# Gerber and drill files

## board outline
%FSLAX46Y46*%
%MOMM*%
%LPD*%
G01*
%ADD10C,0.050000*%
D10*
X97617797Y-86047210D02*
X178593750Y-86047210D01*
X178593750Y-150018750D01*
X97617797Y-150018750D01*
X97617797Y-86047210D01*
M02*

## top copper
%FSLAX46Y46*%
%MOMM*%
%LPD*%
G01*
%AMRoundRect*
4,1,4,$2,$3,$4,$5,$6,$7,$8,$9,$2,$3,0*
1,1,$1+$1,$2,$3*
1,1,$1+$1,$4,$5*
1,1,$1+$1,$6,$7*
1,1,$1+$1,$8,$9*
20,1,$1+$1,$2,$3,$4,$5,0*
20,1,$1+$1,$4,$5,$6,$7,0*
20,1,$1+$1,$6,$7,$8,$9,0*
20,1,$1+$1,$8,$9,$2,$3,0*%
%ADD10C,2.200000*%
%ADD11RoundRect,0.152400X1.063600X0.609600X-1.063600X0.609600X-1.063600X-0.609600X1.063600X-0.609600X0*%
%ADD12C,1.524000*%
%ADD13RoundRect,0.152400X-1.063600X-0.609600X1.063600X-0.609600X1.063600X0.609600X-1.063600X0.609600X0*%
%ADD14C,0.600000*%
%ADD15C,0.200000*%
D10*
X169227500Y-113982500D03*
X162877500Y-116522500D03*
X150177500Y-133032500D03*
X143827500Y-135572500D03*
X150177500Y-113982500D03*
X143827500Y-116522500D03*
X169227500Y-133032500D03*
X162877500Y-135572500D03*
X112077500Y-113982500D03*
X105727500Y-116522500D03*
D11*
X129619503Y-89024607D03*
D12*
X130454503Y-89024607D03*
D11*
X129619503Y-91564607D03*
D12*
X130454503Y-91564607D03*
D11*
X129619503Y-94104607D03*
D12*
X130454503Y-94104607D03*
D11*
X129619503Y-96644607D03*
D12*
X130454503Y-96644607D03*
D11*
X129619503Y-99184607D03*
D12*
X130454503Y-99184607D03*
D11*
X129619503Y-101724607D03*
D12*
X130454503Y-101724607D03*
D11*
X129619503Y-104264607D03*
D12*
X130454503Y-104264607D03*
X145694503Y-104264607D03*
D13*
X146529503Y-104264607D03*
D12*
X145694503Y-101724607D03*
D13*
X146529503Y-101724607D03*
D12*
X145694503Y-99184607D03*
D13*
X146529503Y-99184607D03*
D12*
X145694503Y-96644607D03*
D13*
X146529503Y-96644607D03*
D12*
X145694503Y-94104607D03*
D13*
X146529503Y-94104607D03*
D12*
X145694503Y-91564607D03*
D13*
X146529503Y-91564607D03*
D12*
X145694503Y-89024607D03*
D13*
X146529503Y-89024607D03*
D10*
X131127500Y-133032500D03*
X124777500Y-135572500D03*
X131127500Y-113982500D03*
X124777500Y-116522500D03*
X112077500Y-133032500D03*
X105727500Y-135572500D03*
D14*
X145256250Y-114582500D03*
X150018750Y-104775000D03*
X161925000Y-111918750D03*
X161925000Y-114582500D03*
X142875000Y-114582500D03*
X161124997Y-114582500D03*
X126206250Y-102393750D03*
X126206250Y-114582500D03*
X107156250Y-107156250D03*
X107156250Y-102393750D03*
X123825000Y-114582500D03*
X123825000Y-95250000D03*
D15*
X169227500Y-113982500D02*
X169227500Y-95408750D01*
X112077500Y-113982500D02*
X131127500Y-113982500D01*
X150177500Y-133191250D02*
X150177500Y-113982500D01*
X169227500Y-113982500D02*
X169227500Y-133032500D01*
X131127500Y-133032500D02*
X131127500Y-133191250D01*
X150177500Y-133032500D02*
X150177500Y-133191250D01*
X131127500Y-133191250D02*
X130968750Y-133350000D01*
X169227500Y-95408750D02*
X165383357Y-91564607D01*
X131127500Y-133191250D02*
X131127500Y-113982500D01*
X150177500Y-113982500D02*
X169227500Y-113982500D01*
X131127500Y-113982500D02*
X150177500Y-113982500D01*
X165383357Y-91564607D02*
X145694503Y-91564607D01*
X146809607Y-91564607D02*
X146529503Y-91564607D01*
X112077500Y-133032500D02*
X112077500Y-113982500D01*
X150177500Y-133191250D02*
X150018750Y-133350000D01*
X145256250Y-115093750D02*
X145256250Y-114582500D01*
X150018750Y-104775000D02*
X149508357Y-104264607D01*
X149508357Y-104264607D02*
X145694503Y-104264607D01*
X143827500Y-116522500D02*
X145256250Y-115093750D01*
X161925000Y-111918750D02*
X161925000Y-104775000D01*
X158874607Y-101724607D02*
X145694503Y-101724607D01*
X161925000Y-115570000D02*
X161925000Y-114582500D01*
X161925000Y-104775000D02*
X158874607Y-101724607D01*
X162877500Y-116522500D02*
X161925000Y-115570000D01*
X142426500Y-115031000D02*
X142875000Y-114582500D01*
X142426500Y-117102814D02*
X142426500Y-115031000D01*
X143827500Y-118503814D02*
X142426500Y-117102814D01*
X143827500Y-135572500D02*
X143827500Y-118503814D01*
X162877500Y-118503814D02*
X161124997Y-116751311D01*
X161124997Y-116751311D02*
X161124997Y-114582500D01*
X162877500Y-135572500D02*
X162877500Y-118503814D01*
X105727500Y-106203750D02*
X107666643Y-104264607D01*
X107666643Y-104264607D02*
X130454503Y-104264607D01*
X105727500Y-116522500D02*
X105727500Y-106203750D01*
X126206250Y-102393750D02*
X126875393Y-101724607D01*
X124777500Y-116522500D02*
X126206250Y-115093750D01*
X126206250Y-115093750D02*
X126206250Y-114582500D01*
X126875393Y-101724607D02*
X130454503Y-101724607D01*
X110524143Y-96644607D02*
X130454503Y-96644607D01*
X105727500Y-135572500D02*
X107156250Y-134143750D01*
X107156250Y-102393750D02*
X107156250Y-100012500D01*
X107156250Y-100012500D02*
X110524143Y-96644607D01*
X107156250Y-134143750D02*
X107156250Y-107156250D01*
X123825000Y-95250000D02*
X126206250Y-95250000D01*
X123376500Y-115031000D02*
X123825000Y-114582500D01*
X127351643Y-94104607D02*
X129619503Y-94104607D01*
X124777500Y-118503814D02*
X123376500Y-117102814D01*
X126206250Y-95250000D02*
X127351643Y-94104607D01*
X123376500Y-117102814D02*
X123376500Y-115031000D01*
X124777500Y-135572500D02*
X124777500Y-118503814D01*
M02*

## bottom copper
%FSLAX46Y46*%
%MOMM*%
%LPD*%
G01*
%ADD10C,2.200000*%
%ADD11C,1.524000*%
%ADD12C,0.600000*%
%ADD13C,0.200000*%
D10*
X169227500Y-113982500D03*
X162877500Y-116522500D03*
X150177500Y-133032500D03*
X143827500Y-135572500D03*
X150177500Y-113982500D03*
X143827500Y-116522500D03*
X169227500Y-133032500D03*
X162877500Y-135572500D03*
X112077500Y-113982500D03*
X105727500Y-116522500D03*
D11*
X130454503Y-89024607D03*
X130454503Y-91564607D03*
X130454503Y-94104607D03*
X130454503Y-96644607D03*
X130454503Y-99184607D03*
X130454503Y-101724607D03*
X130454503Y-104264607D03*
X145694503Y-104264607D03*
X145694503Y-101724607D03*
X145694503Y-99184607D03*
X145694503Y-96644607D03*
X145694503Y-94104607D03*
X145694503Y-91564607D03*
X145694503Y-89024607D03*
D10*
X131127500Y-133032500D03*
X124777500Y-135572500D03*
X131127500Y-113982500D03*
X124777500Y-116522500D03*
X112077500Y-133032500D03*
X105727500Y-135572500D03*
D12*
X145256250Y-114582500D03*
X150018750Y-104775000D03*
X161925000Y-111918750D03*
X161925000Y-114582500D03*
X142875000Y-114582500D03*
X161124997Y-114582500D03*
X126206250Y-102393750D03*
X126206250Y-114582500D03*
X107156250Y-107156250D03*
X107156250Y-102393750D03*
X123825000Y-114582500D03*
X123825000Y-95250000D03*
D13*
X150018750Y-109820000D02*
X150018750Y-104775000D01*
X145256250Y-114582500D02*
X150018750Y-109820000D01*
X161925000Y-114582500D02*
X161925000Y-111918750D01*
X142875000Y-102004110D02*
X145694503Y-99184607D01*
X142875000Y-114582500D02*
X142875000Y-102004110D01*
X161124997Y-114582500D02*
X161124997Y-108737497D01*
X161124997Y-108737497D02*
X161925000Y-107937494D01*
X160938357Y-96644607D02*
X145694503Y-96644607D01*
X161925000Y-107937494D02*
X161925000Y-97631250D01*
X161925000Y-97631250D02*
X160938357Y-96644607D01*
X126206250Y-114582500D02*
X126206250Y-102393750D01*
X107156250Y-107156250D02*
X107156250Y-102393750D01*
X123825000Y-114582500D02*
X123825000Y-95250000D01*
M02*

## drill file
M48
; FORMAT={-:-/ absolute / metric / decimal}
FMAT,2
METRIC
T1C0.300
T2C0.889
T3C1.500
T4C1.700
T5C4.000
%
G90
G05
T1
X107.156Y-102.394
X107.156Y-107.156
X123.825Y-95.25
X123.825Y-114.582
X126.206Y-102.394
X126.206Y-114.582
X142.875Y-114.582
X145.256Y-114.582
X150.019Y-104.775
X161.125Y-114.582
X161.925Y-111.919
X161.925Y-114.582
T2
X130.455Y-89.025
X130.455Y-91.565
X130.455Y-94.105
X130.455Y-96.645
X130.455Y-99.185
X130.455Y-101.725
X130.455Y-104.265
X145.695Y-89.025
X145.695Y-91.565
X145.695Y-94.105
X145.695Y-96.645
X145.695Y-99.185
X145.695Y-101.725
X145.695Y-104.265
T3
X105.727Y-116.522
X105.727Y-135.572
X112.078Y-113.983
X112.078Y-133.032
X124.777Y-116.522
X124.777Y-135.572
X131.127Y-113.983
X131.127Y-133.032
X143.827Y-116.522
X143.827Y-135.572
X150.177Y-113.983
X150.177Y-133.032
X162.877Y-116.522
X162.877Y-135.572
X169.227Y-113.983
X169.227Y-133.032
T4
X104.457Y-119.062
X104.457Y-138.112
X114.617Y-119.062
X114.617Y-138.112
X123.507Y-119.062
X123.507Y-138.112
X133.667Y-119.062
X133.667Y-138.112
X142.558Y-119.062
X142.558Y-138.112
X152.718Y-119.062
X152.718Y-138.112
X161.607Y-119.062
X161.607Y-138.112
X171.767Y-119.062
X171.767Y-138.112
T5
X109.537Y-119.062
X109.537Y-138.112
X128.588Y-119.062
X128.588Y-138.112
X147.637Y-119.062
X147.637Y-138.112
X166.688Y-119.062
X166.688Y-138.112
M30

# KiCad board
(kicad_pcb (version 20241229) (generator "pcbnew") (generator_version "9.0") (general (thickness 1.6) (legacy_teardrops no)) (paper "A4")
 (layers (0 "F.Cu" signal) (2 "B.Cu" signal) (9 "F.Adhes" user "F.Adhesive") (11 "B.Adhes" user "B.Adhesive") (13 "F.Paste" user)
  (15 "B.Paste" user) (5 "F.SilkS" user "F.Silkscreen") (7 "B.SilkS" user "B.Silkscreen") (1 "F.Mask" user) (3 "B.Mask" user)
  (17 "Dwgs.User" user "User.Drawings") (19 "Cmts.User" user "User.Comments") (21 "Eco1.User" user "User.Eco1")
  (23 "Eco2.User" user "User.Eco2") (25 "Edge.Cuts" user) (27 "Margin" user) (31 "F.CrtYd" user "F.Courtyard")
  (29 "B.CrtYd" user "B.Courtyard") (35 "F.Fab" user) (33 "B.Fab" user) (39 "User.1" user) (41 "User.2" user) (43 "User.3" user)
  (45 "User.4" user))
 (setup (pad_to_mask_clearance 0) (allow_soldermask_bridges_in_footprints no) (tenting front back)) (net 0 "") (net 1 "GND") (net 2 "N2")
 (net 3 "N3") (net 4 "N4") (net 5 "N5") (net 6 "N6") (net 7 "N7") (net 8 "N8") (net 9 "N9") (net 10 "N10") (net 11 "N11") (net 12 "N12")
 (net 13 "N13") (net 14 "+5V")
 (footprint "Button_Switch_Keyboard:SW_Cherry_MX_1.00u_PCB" (layer "F.Cu") (at 169.2275 113.9825)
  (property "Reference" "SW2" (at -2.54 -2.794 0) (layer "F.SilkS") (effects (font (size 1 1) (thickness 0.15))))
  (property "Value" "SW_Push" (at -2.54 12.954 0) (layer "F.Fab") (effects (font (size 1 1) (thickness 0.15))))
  (pad "" np_thru_hole circle (at -7.62 5.08) (size 1.7 1.7) (drill 1.7) (layers "*.Cu" "*.Mask"))
  (pad "" np_thru_hole circle (at -2.54 5.08) (size 4 4) (drill 4) (layers "*.Cu" "*.Mask"))
  (pad "" np_thru_hole circle (at 2.54 5.08) (size 1.7 1.7) (drill 1.7) (layers "*.Cu" "*.Mask"))
  (pad "1" thru_hole circle (at 0 0) (size 2.2 2.2) (drill 1.5) (layers "*.Cu" "*.Mask") (remove_unused_layers no) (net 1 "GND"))
  (pad "2" thru_hole circle (at -6.35 2.54) (size 2.2 2.2) (drill 1.5) (layers "*.Cu" "*.Mask") (remove_unused_layers no) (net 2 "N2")))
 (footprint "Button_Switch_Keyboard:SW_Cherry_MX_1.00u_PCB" (layer "F.Cu") (at 150.1775 133.0325)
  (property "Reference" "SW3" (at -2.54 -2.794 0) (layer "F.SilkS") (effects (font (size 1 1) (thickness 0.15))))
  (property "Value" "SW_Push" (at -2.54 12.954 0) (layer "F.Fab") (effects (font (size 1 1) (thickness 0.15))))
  (pad "" np_thru_hole circle (at -7.62 5.08) (size 1.7 1.7) (drill 1.7) (layers "*.Cu" "*.Mask"))
  (pad "" np_thru_hole circle (at -2.54 5.08) (size 4 4) (drill 4) (layers "*.Cu" "*.Mask"))
  (pad "" np_thru_hole circle (at 2.54 5.08) (size 1.7 1.7) (drill 1.7) (layers "*.Cu" "*.Mask"))
  (pad "1" thru_hole circle (at 0 0) (size 2.2 2.2) (drill 1.5) (layers "*.Cu" "*.Mask") (remove_unused_layers no) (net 1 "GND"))
  (pad "2" thru_hole circle (at -6.35 2.54) (size 2.2 2.2) (drill 1.5) (layers "*.Cu" "*.Mask") (remove_unused_layers no) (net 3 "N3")))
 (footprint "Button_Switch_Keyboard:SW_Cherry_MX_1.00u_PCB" (layer "F.Cu") (at 150.1775 113.9825)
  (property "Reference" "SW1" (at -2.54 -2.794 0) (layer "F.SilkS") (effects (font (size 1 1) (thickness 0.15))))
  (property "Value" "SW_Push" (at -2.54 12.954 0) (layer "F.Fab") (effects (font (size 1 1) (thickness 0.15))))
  (pad "" np_thru_hole circle (at -7.62 5.08) (size 1.7 1.7) (drill 1.7) (layers "*.Cu" "*.Mask"))
  (pad "" np_thru_hole circle (at -2.54 5.08) (size 4 4) (drill 4) (layers "*.Cu" "*.Mask"))
  (pad "" np_thru_hole circle (at 2.54 5.08) (size 1.7 1.7) (drill 1.7) (layers "*.Cu" "*.Mask"))
  (pad "1" thru_hole circle (at 0 0) (size 2.2 2.2) (drill 1.5) (layers "*.Cu" "*.Mask") (remove_unused_layers no) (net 1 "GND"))
  (pad "2" thru_hole circle (at -6.35 2.54) (size 2.2 2.2) (drill 1.5) (layers "*.Cu" "*.Mask") (remove_unused_layers no) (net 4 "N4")))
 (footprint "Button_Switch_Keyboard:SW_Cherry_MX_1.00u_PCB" (layer "F.Cu") (at 169.2275 133.0325)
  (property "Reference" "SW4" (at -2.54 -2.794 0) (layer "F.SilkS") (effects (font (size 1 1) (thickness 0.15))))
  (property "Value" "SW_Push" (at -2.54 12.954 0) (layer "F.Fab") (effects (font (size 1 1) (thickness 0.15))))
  (pad "" np_thru_hole circle (at -7.62 5.08) (size 1.7 1.7) (drill 1.7) (layers "*.Cu" "*.Mask"))
  (pad "" np_thru_hole circle (at -2.54 5.08) (size 4 4) (drill 4) (layers "*.Cu" "*.Mask"))
  (pad "" np_thru_hole circle (at 2.54 5.08) (size 1.7 1.7) (drill 1.7) (layers "*.Cu" "*.Mask"))
  (pad "1" thru_hole circle (at 0 0) (size 2.2 2.2) (drill 1.5) (layers "*.Cu" "*.Mask") (remove_unused_layers no) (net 1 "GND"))
  (pad "2" thru_hole circle (at -6.35 2.54) (size 2.2 2.2) (drill 1.5) (layers "*.Cu" "*.Mask") (remove_unused_layers no) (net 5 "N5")))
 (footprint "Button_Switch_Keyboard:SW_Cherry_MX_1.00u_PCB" (layer "F.Cu") (at 112.0775 113.9825)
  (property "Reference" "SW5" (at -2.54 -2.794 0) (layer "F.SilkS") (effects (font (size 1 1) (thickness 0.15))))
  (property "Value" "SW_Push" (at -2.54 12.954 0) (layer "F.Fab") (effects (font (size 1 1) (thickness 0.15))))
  (pad "" np_thru_hole circle (at -7.62 5.08) (size 1.7 1.7) (drill 1.7) (layers "*.Cu" "*.Mask"))
  (pad "" np_thru_hole circle (at -2.54 5.08) (size 4 4) (drill 4) (layers "*.Cu" "*.Mask"))
  (pad "" np_thru_hole circle (at 2.54 5.08) (size 1.7 1.7) (drill 1.7) (layers "*.Cu" "*.Mask"))
  (pad "1" thru_hole circle (at 0 0) (size 2.2 2.2) (drill 1.5) (layers "*.Cu" "*.Mask") (remove_unused_layers no) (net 1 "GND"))
  (pad "2" thru_hole circle (at -6.35 2.54) (size 2.2 2.2) (drill 1.5) (layers "*.Cu" "*.Mask") (remove_unused_layers no) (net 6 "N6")))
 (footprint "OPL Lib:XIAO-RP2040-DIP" (layer "F.Cu") (at 138.074503 96.644607)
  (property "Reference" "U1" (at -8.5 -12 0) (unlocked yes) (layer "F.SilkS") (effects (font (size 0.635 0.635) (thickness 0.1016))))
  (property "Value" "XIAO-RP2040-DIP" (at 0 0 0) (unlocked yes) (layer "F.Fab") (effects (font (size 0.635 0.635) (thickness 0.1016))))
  (pad "1" smd roundrect (at -8.455 -7.62 180) (size 2.432 1.524) (layers "F.Cu" "F.Mask") (roundrect_rratio 0.1) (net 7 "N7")
   (thermal_bridge_angle 45))
  (pad "1" thru_hole circle (at -7.62 -7.62 180) (size 1.524 1.524) (drill 0.889) (layers "*.Cu" "*.Mask") (remove_unused_layers no)
   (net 7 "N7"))
  (pad "2" smd roundrect (at -8.455 -5.08 180) (size 2.432 1.524) (layers "F.Cu" "F.Mask") (roundrect_rratio 0.1) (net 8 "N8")
   (thermal_bridge_angle 45))
  (pad "2" thru_hole circle (at -7.62 -5.08 180) (size 1.524 1.524) (drill 0.889) (layers "*.Cu" "*.Mask") (remove_unused_layers no)
   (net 8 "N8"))
  (pad "3" smd roundrect (at -8.455 -2.54 180) (size 2.432 1.524) (layers "F.Cu" "F.Mask") (roundrect_rratio 0.1) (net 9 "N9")
   (thermal_bridge_angle 45))
  (pad "3" thru_hole circle (at -7.62 -2.54 180) (size 1.524 1.524) (drill 0.889) (layers "*.Cu" "*.Mask") (remove_unused_layers no)
   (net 9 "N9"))
  (pad "4" smd roundrect (at -8.455 0 180) (size 2.432 1.524) (layers "F.Cu" "F.Mask") (roundrect_rratio 0.1) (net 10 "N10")
   (thermal_bridge_angle 45))
  (pad "4" thru_hole circle (at -7.62 0 180) (size 1.524 1.524) (drill 0.889) (layers "*.Cu" "*.Mask") (remove_unused_layers no)
   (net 10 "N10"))
  (pad "5" smd roundrect (at -8.455 2.54 180) (size 2.432 1.524) (layers "F.Cu" "F.Mask") (roundrect_rratio 0.1) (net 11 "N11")
   (thermal_bridge_angle 45))
  (pad "5" thru_hole circle (at -7.62 2.54 180) (size 1.524 1.524) (drill 0.889) (layers "*.Cu" "*.Mask") (remove_unused_layers no)
   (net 11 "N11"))
  (pad "6" smd roundrect (at -8.455 5.08 180) (size 2.432 1.524) (layers "F.Cu" "F.Mask") (roundrect_rratio 0.1) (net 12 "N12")
   (thermal_bridge_angle 45))
  (pad "6" thru_hole circle (at -7.62 5.08 180) (size 1.524 1.524) (drill 0.889) (layers "*.Cu" "*.Mask") (remove_unused_layers no)
   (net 12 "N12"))
  (pad "7" smd roundrect (at -8.455 7.62 180) (size 2.432 1.524) (layers "F.Cu" "F.Mask") (roundrect_rratio 0.1) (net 6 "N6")
   (thermal_bridge_angle 45))
  (pad "7" thru_hole circle (at -7.62 7.62 180) (size 1.524 1.524) (drill 0.889) (layers "*.Cu" "*.Mask") (remove_unused_layers no)
   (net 6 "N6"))
  (pad "8" thru_hole circle (at 7.62 7.62) (size 1.524 1.524) (drill 0.889) (layers "*.Cu" "*.Mask") (remove_unused_layers no) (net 4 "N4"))
  (pad "8" smd roundrect (at 8.455 7.62) (size 2.432 1.524) (layers "F.Cu" "F.Mask") (roundrect_rratio 0.1) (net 4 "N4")
   (thermal_bridge_angle 45))
  (pad "9" thru_hole circle (at 7.62 5.08) (size 1.524 1.524) (drill 0.889) (layers "*.Cu" "*.Mask") (remove_unused_layers no) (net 2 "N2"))
  (pad "9" smd roundrect (at 8.455 5.08) (size 2.432 1.524) (layers "F.Cu" "F.Mask") (roundrect_rratio 0.1) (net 2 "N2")
   (thermal_bridge_angle 45))
  (pad "10" thru_hole circle (at 7.62 2.54) (size 1.524 1.524) (drill 0.889) (layers "*.Cu" "*.Mask") (remove_unused_layers no) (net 3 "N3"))
  (pad "10" smd roundrect (at 8.455 2.54) (size 2.432 1.524) (layers "F.Cu" "F.Mask") (roundrect_rratio 0.1) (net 3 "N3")
   (thermal_bridge_angle 45))
  (pad "11" thru_hole circle (at 7.62 0) (size 1.524 1.524) (drill 0.889) (layers "*.Cu" "*.Mask") (remove_unused_layers no) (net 5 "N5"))
  (pad "11" smd roundrect (at 8.455 0) (size 2.432 1.524) (layers "F.Cu" "F.Mask") (roundrect_rratio 0.1) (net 5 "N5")
   (thermal_bridge_angle 45))
  (pad "12" thru_hole circle (at 7.62 -2.54) (size 1.524 1.524) (drill 0.889) (layers "*.Cu" "*.Mask") (remove_unused_layers no)
   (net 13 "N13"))
  (pad "12" smd roundrect (at 8.455 -2.54) (size 2.432 1.524) (layers "F.Cu" "F.Mask") (roundrect_rratio 0.1) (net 13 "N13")
   (thermal_bridge_angle 45))
  (pad "13" thru_hole circle (at 7.62 -5.08) (size 1.524 1.524) (drill 0.889) (layers "*.Cu" "*.Mask") (remove_unused_layers no)
   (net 1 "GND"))
  (pad "13" smd roundrect (at 8.455 -5.08) (size 2.432 1.524) (layers "F.Cu" "F.Mask") (roundrect_rratio 0.1) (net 1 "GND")
   (thermal_bridge_angle 45))
  (pad "14" thru_hole circle (at 7.62 -7.62) (size 1.524 1.524) (drill 0.889) (layers "*.Cu" "*.Mask") (remove_unused_layers no)
   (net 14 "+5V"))
  (pad "14" smd roundrect (at 8.455 -7.62) (size 2.432 1.524) (layers "F.Cu" "F.Mask") (roundrect_rratio 0.1) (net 14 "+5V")
   (thermal_bridge_angle 45)))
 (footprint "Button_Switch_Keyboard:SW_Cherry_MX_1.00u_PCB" (layer "F.Cu") (at 131.1275 133.0325)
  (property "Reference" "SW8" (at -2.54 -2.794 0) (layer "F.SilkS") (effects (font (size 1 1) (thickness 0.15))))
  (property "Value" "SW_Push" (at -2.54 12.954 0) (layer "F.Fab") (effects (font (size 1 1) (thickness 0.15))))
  (pad "" np_thru_hole circle (at -7.62 5.08) (size 1.7 1.7) (drill 1.7) (layers "*.Cu" "*.Mask"))
  (pad "" np_thru_hole circle (at -2.54 5.08) (size 4 4) (drill 4) (layers "*.Cu" "*.Mask"))
  (pad "" np_thru_hole circle (at 2.54 5.08) (size 1.7 1.7) (drill 1.7) (layers "*.Cu" "*.Mask"))
  (pad "1" thru_hole circle (at 0 0) (size 2.2 2.2) (drill 1.5) (layers "*.Cu" "*.Mask") (remove_unused_layers no) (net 1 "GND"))
  (pad "2" thru_hole circle (at -6.35 2.54) (size 2.2 2.2) (drill 1.5) (layers "*.Cu" "*.Mask") (remove_unused_layers no) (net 9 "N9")))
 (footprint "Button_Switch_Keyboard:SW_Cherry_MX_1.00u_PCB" (layer "F.Cu") (at 131.1275 113.9825)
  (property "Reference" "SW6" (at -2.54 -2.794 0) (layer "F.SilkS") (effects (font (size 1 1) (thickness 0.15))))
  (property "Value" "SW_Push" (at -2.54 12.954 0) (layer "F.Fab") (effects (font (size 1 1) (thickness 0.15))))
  (pad "" np_thru_hole circle (at -7.62 5.08) (size 1.7 1.7) (drill 1.7) (layers "*.Cu" "*.Mask"))
  (pad "" np_thru_hole circle (at -2.54 5.08) (size 4 4) (drill 4) (layers "*.Cu" "*.Mask"))
  (pad "" np_thru_hole circle (at 2.54 5.08) (size 1.7 1.7) (drill 1.7) (layers "*.Cu" "*.Mask"))
  (pad "1" thru_hole circle (at 0 0) (size 2.2 2.2) (drill 1.5) (layers "*.Cu" "*.Mask") (remove_unused_layers no) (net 1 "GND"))
  (pad "2" thru_hole circle (at -6.35 2.54) (size 2.2 2.2) (drill 1.5) (layers "*.Cu" "*.Mask") (remove_unused_layers no) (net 12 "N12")))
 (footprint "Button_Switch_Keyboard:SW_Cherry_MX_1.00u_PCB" (layer "F.Cu") (at 112.0775 133.0325)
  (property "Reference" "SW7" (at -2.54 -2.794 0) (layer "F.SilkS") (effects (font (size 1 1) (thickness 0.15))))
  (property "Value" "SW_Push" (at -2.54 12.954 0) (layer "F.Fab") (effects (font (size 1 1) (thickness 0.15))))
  (pad "" np_thru_hole circle (at -7.62 5.08) (size 1.7 1.7) (drill 1.7) (layers "*.Cu" "*.Mask"))
  (pad "" np_thru_hole circle (at -2.54 5.08) (size 4 4) (drill 4) (layers "*.Cu" "*.Mask"))
  (pad "" np_thru_hole circle (at 2.54 5.08) (size 1.7 1.7) (drill 1.7) (layers "*.Cu" "*.Mask"))
  (pad "1" thru_hole circle (at 0 0) (size 2.2 2.2) (drill 1.5) (layers "*.Cu" "*.Mask") (remove_unused_layers no) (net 1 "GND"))
  (pad "2" thru_hole circle (at -6.35 2.54) (size 2.2 2.2) (drill 1.5) (layers "*.Cu" "*.Mask") (remove_unused_layers no) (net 10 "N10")))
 (gr_rect (start 97.617797 86.04721) (end 178.59375 150.01875) (stroke (width 0.05) (type default)) (fill no) (layer "Edge.Cuts"))
 (segment (start 169.2275 113.9825) (end 169.2275 95.40875) (width 0.2) (layer "F.Cu") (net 1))
 (segment (start 112.0775 113.9825) (end 131.1275 113.9825) (width 0.2) (layer "F.Cu") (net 1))
 (segment (start 150.1775 133.19125) (end 150.1775 113.9825) (width 0.2) (layer "F.Cu") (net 1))
 (segment (start 169.2275 113.9825) (end 169.2275 133.0325) (width 0.2) (layer "F.Cu") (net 1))
 (segment (start 131.1275 133.0325) (end 131.1275 133.19125) (width 0.2) (layer "F.Cu") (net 1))
 (segment (start 150.1775 133.0325) (end 150.1775 133.19125) (width 0.2) (layer "F.Cu") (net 1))
 (segment (start 131.1275 133.19125) (end 130.96875 133.35) (width 0.2) (layer "F.Cu") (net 1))
 (segment (start 169.2275 95.40875) (end 165.383357 91.564607) (width 0.2) (layer "F.Cu") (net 1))
 (segment (start 131.1275 133.19125) (end 131.1275 113.9825) (width 0.2) (layer "F.Cu") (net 1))
 (segment (start 150.1775 113.9825) (end 169.2275 113.9825) (width 0.2) (layer "F.Cu") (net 1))
 (segment (start 131.1275 113.9825) (end 150.1775 113.9825) (width 0.2) (layer "F.Cu") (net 1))
 (segment (start 165.383357 91.564607) (end 145.694503 91.564607) (width 0.2) (layer "F.Cu") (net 1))
 (segment (start 146.809607 91.564607) (end 146.529503 91.564607) (width 0.2) (layer "F.Cu") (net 1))
 (segment (start 112.0775 133.0325) (end 112.0775 113.9825) (width 0.2) (layer "F.Cu") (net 1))
 (segment (start 150.1775 133.19125) (end 150.01875 133.35) (width 0.2) (layer "F.Cu") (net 1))
 (segment (start 145.25625 115.09375) (end 145.25625 114.5825) (width 0.2) (layer "F.Cu") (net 4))
 (segment (start 150.01875 104.775) (end 149.508357 104.264607) (width 0.2) (layer "F.Cu") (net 4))
 (segment (start 149.508357 104.264607) (end 145.694503 104.264607) (width 0.2) (layer "F.Cu") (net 4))
 (segment (start 143.8275 116.5225) (end 145.25625 115.09375) (width 0.2) (layer "F.Cu") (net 4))
 (via (at 145.25625 114.5825) (size 0.6) (drill 0.3) (layers "F.Cu" "B.Cu") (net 4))
 (via (at 150.01875 104.775) (size 0.6) (drill 0.3) (layers "F.Cu" "B.Cu") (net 4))
 (segment (start 150.01875 109.82) (end 150.01875 104.775) (width 0.2) (layer "B.Cu") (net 4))
 (segment (start 145.25625 114.5825) (end 150.01875 109.82) (width 0.2) (layer "B.Cu") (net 4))
 (segment (start 161.925 111.91875) (end 161.925 104.775) (width 0.2) (layer "F.Cu") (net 2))
 (segment (start 158.874607 101.724607) (end 145.694503 101.724607) (width 0.2) (layer "F.Cu") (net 2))
 (segment (start 161.925 115.57) (end 161.925 114.5825) (width 0.2) (layer "F.Cu") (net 2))
 (segment (start 161.925 104.775) (end 158.874607 101.724607) (width 0.2) (layer "F.Cu") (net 2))
 (segment (start 162.8775 116.5225) (end 161.925 115.57) (width 0.2) (layer "F.Cu") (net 2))
 (via (at 161.925 111.91875) (size 0.6) (drill 0.3) (layers "F.Cu" "B.Cu") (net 2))
 (via (at 161.925 114.5825) (size 0.6) (drill 0.3) (layers "F.Cu" "B.Cu") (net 2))
 (segment (start 161.925 114.5825) (end 161.925 111.91875) (width 0.2) (layer "B.Cu") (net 2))
 (segment (start 142.4265 115.031) (end 142.875 114.5825) (width 0.2) (layer "F.Cu") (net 3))
 (segment (start 142.4265 117.102814) (end 142.4265 115.031) (width 0.2) (layer "F.Cu") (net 3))
 (segment (start 143.8275 118.503814) (end 142.4265 117.102814) (width 0.2) (layer "F.Cu") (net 3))
 (segment (start 143.8275 135.5725) (end 143.8275 118.503814) (width 0.2) (layer "F.Cu") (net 3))
 (via (at 142.875 114.5825) (size 0.6) (drill 0.3) (layers "F.Cu" "B.Cu") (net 3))
 (segment (start 142.875 102.00411) (end 145.694503 99.184607) (width 0.2) (layer "B.Cu") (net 3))
 (segment (start 142.875 114.5825) (end 142.875 102.00411) (width 0.2) (layer "B.Cu") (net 3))
 (segment (start 162.8775 118.503814) (end 161.124997 116.751311) (width 0.2) (layer "F.Cu") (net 5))
 (segment (start 161.124997 116.751311) (end 161.124997 114.5825) (width 0.2) (layer "F.Cu") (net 5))
 (segment (start 162.8775 135.5725) (end 162.8775 118.503814) (width 0.2) (layer "F.Cu") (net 5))
 (via (at 161.124997 114.5825) (size 0.6) (drill 0.3) (layers "F.Cu" "B.Cu") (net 5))
 (segment (start 161.124997 114.5825) (end 161.124997 108.737497) (width 0.2) (layer "B.Cu") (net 5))
 (segment (start 161.124997 108.737497) (end 161.925 107.937494) (width 0.2) (layer "B.Cu") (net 5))
 (segment (start 160.938357 96.644607) (end 145.694503 96.644607) (width 0.2) (layer "B.Cu") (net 5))
 (segment (start 161.925 107.937494) (end 161.925 97.63125) (width 0.2) (layer "B.Cu") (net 5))
 (segment (start 161.925 97.63125) (end 160.938357 96.644607) (width 0.2) (layer "B.Cu") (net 5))
 (segment (start 105.7275 106.20375) (end 107.666643 104.264607) (width 0.2) (layer "F.Cu") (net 6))
 (segment (start 107.666643 104.264607) (end 130.454503 104.264607) (width 0.2) (layer "F.Cu") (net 6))
 (segment (start 105.7275 116.5225) (end 105.7275 106.20375) (width 0.2) (layer "F.Cu") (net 6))
 (segment (start 126.20625 102.39375) (end 126.875393 101.724607) (width 0.2) (layer "F.Cu") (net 12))
 (segment (start 124.7775 116.5225) (end 126.20625 115.09375) (width 0.2) (layer "F.Cu") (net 12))
 (segment (start 126.20625 115.09375) (end 126.20625 114.5825) (width 0.2) (layer "F.Cu") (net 12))
 (segment (start 126.875393 101.724607) (end 130.454503 101.724607) (width 0.2) (layer "F.Cu") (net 12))
 (via (at 126.20625 102.39375) (size 0.6) (drill 0.3) (layers "F.Cu" "B.Cu") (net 12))
 (via (at 126.20625 114.5825) (size 0.6) (drill 0.3) (layers "F.Cu" "B.Cu") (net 12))
 (segment (start 126.20625 114.5825) (end 126.20625 102.39375) (width 0.2) (layer "B.Cu") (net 12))
 (segment (start 110.524143 96.644607) (end 130.454503 96.644607) (width 0.2) (layer "F.Cu") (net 10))
 (segment (start 105.7275 135.5725) (end 107.15625 134.14375) (width 0.2) (layer "F.Cu") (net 10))
 (segment (start 107.15625 102.39375) (end 107.15625 100.0125) (width 0.2) (layer "F.Cu") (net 10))
 (segment (start 107.15625 100.0125) (end 110.524143 96.644607) (width 0.2) (layer "F.Cu") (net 10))
 (segment (start 107.15625 134.14375) (end 107.15625 107.15625) (width 0.2) (layer "F.Cu") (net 10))
 (via (at 107.15625 107.15625) (size 0.6) (drill 0.3) (layers "F.Cu" "B.Cu") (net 10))
 (via (at 107.15625 102.39375) (size 0.6) (drill 0.3) (layers "F.Cu" "B.Cu") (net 10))
 (segment (start 107.15625 107.15625) (end 107.15625 102.39375) (width 0.2) (layer "B.Cu") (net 10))
 (segment (start 123.825 95.25) (end 126.20625 95.25) (width 0.2) (layer "F.Cu") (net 9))
 (segment (start 123.3765 115.031) (end 123.825 114.5825) (width 0.2) (layer "F.Cu") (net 9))
 (segment (start 127.351643 94.104607) (end 129.619503 94.104607) (width 0.2) (layer "F.Cu") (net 9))
 (segment (start 124.7775 118.503814) (end 123.3765 117.102814) (width 0.2) (layer "F.Cu") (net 9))
 (segment (start 126.20625 95.25) (end 127.351643 94.104607) (width 0.2) (layer "F.Cu") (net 9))
 (segment (start 123.3765 117.102814) (end 123.3765 115.031) (width 0.2) (layer "F.Cu") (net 9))
 (segment (start 124.7775 135.5725) (end 124.7775 118.503814) (width 0.2) (layer "F.Cu") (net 9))
 (via (at 123.825 114.5825) (size 0.6) (drill 0.3) (layers "F.Cu" "B.Cu") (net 9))
 (via (at 123.825 95.25) (size 0.6) (drill 0.3) (layers "F.Cu" "B.Cu") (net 9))
 (segment (start 123.825 114.5825) (end 123.825 95.25) (width 0.2) (layer "B.Cu") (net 9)))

